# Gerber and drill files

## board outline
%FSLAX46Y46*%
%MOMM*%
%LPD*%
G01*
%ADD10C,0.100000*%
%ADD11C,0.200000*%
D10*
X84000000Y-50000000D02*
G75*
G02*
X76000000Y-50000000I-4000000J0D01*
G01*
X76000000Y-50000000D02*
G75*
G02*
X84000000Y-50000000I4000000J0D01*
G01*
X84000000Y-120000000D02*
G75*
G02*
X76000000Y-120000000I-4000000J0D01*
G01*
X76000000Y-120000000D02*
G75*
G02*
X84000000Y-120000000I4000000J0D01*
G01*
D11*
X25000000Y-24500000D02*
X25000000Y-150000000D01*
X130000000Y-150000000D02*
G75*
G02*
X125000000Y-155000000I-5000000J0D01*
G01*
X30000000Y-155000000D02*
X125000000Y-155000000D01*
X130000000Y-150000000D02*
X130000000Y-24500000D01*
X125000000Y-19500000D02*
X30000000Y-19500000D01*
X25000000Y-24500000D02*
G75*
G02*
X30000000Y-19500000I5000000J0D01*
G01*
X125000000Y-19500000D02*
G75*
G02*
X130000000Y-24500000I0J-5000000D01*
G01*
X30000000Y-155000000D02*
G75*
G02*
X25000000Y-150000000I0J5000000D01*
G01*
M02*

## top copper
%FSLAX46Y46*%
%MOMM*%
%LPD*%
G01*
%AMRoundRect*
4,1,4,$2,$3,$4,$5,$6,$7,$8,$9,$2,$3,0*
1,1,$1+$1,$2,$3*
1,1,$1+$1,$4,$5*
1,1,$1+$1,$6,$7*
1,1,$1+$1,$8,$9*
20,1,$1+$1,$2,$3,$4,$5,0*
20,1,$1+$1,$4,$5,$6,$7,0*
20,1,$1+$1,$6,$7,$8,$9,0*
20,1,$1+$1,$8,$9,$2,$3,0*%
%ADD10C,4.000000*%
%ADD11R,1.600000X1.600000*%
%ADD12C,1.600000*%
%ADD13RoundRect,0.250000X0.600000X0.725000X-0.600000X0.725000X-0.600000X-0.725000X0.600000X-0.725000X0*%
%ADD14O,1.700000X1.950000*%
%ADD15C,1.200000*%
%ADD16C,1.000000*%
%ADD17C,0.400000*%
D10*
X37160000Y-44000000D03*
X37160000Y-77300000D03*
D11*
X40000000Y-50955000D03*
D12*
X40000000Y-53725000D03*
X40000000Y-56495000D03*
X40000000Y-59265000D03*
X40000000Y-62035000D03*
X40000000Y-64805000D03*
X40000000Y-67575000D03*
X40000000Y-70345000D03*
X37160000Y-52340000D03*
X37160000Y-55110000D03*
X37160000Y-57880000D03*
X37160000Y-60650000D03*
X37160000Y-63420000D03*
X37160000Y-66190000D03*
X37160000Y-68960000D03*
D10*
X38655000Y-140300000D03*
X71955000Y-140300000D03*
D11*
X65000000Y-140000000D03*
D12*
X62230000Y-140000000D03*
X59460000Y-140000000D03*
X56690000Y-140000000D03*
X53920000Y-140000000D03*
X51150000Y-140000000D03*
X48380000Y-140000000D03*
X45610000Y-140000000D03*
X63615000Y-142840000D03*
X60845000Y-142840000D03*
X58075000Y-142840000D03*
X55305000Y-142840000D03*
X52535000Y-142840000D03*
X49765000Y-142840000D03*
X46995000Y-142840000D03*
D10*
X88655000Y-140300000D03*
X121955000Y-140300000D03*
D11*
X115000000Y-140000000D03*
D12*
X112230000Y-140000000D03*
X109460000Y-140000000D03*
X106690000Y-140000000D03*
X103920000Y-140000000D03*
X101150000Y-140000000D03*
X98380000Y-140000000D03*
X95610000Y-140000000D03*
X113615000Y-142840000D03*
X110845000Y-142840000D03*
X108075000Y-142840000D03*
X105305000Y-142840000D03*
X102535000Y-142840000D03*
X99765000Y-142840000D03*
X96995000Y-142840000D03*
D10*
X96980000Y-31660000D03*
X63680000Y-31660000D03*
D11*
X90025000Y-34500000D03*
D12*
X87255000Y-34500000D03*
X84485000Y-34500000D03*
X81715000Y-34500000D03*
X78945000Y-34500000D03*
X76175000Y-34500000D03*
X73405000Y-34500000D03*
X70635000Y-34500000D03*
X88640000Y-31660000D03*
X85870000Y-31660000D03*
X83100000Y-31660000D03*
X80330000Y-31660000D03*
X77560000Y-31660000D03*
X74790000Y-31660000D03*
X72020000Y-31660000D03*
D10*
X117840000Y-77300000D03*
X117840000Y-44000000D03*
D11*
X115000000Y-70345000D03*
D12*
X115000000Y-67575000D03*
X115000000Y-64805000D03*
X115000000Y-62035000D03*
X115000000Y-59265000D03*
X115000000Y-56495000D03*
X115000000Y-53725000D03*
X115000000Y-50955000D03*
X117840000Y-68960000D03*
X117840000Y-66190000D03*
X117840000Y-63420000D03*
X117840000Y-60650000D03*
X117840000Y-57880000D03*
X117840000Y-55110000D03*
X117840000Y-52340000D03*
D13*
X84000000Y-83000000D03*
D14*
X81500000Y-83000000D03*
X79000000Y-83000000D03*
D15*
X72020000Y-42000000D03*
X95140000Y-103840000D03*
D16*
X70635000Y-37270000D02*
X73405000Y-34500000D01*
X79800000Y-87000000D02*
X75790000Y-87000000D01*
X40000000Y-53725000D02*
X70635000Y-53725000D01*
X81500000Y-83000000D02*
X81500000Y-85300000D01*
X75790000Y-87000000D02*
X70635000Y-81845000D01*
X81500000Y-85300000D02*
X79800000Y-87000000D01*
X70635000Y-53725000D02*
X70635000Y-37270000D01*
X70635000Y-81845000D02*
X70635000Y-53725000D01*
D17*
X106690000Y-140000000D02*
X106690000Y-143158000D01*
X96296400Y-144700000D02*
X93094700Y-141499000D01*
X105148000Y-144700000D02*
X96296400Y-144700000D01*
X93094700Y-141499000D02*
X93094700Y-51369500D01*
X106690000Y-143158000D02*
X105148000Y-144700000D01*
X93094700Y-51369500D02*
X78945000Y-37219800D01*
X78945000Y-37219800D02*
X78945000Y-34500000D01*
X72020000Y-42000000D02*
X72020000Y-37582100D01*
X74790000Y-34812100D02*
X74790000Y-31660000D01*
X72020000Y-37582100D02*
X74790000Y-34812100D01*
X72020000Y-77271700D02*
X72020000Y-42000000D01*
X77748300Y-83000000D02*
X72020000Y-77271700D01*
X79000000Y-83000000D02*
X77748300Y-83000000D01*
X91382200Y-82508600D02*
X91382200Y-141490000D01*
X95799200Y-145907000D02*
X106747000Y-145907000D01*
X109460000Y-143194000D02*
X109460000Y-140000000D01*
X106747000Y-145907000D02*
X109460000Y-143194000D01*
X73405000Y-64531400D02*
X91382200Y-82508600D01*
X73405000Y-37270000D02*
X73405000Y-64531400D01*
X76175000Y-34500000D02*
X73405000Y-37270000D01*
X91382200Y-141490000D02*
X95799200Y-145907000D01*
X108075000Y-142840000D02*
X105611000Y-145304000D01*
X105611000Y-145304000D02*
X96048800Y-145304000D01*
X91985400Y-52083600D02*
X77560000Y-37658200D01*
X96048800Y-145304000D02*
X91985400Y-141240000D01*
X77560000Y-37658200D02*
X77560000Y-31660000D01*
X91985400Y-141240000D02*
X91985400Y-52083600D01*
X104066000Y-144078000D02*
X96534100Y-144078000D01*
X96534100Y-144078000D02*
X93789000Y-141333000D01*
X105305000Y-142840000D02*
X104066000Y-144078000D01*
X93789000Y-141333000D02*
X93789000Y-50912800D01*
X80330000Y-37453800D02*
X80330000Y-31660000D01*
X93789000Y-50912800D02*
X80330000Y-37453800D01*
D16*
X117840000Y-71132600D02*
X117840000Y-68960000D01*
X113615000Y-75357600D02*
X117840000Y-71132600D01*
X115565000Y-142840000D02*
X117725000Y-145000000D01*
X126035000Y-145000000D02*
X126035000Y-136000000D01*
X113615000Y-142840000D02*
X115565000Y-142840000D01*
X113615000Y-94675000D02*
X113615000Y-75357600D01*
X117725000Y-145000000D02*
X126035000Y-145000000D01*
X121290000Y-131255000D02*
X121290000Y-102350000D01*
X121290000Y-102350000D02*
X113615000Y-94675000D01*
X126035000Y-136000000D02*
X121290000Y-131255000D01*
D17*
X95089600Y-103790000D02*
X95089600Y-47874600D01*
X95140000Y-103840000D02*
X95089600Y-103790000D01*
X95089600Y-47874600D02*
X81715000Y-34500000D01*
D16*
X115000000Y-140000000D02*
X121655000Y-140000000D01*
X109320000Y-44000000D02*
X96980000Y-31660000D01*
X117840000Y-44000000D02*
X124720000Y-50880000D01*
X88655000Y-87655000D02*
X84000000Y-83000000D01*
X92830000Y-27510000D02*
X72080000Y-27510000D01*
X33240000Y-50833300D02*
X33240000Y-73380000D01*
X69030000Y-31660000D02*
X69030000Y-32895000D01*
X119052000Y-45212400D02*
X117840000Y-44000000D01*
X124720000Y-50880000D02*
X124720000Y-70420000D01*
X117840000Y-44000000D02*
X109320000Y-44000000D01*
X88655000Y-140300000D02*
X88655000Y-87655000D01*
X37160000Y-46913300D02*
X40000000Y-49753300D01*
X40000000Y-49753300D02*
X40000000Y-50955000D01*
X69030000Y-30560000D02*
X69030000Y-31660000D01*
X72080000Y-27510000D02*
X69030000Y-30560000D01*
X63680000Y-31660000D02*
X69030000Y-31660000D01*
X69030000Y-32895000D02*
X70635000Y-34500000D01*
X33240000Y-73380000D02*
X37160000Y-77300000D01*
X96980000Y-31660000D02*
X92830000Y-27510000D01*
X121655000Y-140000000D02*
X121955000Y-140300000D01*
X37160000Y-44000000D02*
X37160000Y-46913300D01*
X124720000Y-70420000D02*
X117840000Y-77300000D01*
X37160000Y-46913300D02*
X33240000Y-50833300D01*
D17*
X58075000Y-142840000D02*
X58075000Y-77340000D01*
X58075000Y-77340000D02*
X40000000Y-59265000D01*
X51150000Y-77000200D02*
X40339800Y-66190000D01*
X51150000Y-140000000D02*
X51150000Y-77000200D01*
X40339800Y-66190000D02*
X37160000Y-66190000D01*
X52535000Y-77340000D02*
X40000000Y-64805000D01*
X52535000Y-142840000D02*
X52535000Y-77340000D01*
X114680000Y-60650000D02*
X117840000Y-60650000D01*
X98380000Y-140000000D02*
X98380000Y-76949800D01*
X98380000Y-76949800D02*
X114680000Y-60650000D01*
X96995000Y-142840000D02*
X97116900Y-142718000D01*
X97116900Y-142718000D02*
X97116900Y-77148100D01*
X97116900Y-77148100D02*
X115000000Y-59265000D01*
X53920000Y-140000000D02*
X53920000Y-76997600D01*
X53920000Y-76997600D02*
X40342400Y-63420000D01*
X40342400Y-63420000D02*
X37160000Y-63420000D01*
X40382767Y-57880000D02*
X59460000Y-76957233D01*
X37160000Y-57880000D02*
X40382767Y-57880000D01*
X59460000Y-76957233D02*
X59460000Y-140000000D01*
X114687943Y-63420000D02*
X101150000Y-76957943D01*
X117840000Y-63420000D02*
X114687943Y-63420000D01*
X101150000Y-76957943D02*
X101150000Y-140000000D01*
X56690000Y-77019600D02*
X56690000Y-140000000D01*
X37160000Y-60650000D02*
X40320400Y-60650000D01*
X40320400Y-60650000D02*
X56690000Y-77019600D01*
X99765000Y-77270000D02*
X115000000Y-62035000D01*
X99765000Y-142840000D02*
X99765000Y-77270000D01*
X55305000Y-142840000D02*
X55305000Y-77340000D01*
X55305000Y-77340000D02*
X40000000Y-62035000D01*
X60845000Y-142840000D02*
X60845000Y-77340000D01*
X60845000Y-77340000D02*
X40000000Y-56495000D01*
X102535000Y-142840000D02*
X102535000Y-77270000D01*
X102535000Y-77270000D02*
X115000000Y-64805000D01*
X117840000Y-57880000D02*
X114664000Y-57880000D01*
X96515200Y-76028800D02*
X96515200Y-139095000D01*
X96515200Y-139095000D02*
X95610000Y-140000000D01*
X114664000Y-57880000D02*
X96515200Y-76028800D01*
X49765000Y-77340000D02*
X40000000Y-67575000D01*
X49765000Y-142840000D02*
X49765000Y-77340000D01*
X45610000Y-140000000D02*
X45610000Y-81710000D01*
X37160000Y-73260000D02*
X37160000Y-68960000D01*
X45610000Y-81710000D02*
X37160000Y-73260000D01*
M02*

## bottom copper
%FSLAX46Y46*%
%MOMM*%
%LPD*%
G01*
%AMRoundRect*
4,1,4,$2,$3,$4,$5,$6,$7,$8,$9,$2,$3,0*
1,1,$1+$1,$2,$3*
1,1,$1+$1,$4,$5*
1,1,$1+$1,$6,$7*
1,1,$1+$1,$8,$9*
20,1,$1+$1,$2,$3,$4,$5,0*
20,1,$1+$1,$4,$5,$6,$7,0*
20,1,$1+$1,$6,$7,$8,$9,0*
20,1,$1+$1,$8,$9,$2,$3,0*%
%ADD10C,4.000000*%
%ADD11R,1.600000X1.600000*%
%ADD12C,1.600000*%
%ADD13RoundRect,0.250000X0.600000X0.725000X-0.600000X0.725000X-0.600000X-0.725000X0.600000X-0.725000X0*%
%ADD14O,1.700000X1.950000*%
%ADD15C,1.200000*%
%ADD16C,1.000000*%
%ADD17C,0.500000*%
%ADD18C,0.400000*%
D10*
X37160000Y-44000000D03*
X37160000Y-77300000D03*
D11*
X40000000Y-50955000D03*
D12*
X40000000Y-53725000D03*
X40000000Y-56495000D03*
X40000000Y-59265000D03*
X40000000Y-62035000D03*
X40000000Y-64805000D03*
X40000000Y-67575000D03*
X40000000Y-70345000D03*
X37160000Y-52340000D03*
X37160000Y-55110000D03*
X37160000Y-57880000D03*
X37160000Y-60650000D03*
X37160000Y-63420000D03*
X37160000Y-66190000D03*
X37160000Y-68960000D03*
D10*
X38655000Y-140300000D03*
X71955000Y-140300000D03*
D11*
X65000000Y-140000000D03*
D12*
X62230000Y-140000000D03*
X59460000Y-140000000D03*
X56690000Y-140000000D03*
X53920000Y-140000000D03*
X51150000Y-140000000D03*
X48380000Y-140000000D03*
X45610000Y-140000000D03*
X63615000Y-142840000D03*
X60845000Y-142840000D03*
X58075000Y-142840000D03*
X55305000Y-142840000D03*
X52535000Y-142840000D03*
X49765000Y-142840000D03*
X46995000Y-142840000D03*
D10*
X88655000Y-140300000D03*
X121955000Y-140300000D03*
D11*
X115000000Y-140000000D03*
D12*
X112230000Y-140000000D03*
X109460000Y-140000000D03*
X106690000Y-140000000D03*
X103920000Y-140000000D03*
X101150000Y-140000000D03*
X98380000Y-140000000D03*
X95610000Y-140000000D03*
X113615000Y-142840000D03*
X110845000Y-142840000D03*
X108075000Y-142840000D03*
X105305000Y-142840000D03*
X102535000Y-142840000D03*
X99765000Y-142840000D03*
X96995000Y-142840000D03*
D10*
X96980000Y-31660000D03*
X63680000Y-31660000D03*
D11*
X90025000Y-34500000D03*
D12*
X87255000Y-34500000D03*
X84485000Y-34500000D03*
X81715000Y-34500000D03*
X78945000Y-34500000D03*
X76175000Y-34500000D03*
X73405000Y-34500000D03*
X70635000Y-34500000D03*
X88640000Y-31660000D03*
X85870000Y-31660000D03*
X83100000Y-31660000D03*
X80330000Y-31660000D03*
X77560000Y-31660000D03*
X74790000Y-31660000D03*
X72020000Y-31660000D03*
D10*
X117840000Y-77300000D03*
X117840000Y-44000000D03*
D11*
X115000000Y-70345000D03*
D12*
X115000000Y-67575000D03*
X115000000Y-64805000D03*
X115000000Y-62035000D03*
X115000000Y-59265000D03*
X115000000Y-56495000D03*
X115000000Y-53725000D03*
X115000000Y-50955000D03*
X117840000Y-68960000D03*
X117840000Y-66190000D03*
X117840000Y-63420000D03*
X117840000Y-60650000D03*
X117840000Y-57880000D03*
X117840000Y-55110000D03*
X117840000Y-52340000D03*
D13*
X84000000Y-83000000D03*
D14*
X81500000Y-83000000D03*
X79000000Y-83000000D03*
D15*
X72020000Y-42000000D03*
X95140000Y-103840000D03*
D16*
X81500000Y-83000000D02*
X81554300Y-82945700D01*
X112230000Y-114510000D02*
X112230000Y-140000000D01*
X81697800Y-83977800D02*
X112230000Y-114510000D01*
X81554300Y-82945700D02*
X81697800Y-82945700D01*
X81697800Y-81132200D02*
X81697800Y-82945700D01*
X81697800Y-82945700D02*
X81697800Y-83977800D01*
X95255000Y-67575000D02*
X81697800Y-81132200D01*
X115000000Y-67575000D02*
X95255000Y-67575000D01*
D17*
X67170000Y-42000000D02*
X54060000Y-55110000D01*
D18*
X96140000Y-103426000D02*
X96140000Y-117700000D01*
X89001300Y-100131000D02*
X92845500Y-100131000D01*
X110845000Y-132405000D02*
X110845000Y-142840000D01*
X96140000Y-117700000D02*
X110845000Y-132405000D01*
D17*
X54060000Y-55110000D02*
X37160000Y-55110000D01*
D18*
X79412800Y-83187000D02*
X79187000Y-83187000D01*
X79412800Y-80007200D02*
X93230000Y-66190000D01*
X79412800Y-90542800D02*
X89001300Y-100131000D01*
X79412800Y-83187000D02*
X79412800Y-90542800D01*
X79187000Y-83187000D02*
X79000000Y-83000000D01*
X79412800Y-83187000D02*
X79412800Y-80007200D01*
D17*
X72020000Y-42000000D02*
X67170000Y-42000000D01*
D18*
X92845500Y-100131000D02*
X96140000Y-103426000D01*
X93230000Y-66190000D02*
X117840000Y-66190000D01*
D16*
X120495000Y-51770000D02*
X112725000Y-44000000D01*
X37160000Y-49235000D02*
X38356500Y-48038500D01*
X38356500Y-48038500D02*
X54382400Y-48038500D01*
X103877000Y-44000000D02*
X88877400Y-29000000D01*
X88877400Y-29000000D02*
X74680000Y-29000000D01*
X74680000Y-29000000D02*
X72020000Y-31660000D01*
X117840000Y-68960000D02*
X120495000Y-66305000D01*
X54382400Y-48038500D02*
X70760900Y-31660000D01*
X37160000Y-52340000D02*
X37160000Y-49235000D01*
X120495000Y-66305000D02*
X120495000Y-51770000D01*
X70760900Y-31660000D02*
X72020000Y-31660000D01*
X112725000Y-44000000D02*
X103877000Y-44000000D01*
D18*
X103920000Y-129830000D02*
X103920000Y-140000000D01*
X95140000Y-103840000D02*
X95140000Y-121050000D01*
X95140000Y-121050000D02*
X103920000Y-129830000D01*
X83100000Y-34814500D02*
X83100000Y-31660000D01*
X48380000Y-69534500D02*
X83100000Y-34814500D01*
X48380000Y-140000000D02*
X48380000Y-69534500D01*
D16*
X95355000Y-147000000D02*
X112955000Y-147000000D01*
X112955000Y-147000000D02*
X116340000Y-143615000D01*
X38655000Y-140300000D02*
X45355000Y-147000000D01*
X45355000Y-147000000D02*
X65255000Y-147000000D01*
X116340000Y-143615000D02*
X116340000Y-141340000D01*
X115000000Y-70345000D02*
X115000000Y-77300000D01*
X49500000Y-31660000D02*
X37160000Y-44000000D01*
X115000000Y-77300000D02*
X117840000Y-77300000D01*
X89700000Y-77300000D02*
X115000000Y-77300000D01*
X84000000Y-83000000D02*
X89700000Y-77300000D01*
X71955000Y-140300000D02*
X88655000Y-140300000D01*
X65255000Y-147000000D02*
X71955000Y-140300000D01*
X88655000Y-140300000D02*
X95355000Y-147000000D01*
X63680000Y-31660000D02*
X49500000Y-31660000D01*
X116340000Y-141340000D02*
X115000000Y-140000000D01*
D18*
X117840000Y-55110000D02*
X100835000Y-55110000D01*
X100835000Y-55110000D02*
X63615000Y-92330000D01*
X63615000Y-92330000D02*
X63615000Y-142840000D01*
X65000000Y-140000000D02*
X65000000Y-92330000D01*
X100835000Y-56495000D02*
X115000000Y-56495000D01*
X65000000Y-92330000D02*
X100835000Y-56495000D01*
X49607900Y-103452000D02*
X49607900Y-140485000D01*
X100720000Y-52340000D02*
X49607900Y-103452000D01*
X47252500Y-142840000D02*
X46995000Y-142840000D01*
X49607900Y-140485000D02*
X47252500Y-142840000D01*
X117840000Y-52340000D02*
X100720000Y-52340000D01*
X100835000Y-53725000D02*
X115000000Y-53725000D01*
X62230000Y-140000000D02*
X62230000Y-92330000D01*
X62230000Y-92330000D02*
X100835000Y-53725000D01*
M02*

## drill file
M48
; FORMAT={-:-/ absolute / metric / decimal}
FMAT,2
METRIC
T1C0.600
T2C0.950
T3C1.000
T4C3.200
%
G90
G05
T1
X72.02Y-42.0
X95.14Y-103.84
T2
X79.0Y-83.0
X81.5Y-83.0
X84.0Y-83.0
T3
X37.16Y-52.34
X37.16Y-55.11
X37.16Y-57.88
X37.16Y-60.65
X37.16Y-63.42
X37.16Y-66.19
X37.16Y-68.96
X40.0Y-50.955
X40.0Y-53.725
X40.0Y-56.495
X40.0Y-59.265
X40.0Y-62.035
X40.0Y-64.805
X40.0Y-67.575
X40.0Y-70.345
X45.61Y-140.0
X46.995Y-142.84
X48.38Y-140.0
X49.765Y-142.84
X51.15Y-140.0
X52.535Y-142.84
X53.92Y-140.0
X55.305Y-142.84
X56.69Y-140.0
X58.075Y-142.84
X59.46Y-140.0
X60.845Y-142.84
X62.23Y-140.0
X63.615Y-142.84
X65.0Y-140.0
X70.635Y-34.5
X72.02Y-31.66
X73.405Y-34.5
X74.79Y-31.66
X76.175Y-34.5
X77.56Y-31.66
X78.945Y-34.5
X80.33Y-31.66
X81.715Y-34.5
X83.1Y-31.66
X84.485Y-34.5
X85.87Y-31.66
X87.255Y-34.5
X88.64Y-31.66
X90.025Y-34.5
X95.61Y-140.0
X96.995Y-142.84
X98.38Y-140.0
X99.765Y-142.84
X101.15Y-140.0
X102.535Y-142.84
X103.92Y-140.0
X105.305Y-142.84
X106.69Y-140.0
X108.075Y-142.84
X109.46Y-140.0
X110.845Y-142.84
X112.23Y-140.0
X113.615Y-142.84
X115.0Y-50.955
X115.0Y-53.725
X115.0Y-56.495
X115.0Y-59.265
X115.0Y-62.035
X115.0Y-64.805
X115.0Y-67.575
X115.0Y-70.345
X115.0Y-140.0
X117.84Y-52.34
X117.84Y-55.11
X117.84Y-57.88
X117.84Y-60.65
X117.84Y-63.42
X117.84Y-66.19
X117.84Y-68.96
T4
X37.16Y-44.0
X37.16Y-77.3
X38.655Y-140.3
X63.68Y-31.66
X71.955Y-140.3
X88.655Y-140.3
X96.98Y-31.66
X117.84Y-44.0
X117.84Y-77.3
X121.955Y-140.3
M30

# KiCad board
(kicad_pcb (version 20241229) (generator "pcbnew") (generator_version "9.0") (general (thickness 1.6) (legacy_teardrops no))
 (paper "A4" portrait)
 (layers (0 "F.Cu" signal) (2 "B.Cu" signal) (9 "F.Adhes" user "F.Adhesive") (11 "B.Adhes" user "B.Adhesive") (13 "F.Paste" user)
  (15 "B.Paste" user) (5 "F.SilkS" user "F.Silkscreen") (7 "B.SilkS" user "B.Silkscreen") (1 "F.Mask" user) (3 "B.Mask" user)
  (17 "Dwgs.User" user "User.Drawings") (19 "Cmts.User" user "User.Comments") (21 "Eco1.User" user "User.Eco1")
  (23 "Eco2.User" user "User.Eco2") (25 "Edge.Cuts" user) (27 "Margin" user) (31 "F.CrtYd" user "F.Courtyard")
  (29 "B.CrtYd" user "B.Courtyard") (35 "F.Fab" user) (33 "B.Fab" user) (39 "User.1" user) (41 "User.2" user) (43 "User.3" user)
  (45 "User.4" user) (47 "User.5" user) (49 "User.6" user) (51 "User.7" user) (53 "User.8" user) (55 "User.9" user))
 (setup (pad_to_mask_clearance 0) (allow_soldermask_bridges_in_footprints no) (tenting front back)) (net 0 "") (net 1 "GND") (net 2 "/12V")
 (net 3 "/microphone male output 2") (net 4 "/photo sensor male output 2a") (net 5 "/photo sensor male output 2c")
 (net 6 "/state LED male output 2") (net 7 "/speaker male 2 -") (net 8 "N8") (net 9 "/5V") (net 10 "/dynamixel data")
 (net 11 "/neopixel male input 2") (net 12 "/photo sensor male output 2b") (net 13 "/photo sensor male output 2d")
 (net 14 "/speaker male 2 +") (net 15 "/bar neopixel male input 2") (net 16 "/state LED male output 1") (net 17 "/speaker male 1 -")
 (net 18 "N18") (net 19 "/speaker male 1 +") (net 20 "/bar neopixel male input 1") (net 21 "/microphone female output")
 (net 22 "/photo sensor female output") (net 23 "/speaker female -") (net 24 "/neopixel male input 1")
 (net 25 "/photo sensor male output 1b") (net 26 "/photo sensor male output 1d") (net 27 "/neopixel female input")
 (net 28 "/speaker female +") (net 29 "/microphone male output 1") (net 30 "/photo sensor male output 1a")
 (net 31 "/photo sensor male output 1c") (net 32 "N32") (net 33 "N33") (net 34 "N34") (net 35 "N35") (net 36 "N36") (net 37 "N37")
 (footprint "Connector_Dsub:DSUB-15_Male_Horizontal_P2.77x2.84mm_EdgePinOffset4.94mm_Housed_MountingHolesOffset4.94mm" (layer "F.Cu")
  (at 40 50.955 -90)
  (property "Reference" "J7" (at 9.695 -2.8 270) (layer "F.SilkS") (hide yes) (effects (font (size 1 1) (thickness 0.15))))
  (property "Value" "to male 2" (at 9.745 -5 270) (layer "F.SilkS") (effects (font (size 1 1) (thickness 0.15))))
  (pad "0" thru_hole circle (at -6.955 2.84 270) (size 4 4) (drill 3.2) (layers "*.Cu" "*.Mask") (remove_unused_layers no) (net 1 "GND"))
  (pad "0" thru_hole circle (at 26.345 2.84 270) (size 4 4) (drill 3.2) (layers "*.Cu" "*.Mask") (remove_unused_layers no) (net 1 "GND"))
  (pad "1" thru_hole rect (at 0 0 270) (size 1.6 1.6) (drill 1) (layers "*.Cu" "*.Mask") (remove_unused_layers no) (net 1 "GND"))
  (pad "2" thru_hole circle (at 2.77 0 270) (size 1.6 1.6) (drill 1) (layers "*.Cu" "*.Mask") (remove_unused_layers no) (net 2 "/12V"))
  (pad "3" thru_hole circle (at 5.54 0 270) (size 1.6 1.6) (drill 1) (layers "*.Cu" "*.Mask") (remove_unused_layers no)
   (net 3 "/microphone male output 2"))
  (pad "4" thru_hole circle (at 8.31 0 270) (size 1.6 1.6) (drill 1) (layers "*.Cu" "*.Mask") (remove_unused_layers no)
   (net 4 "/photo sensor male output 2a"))
  (pad "5" thru_hole circle (at 11.08 0 270) (size 1.6 1.6) (drill 1) (layers "*.Cu" "*.Mask") (remove_unused_layers no)
   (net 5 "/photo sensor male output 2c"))
  (pad "6" thru_hole circle (at 13.85 0 270) (size 1.6 1.6) (drill 1) (layers "*.Cu" "*.Mask") (remove_unused_layers no)
   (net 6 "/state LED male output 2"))
  (pad "7" thru_hole circle (at 16.62 0 270) (size 1.6 1.6) (drill 1) (layers "*.Cu" "*.Mask") (remove_unused_layers no)
   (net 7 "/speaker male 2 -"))
  (pad "8" thru_hole circle (at 19.39 0 270) (size 1.6 1.6) (drill 1) (layers "*.Cu" "*.Mask") (remove_unused_layers no) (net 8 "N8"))
  (pad "9" thru_hole circle (at 1.385 2.84 270) (size 1.6 1.6) (drill 1) (layers "*.Cu" "*.Mask") (remove_unused_layers no) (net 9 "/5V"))
  (pad "10" thru_hole circle (at 4.155 2.84 270) (size 1.6 1.6) (drill 1) (layers "*.Cu" "*.Mask") (remove_unused_layers no)
   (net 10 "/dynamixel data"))
  (pad "11" thru_hole circle (at 6.925 2.84 270) (size 1.6 1.6) (drill 1) (layers "*.Cu" "*.Mask") (remove_unused_layers no)
   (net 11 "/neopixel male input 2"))
  (pad "12" thru_hole circle (at 9.695 2.84 270) (size 1.6 1.6) (drill 1) (layers "*.Cu" "*.Mask") (remove_unused_layers no)
   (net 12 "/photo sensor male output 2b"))
  (pad "13" thru_hole circle (at 12.465 2.84 270) (size 1.6 1.6) (drill 1) (layers "*.Cu" "*.Mask") (remove_unused_layers no)
   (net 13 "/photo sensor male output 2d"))
  (pad "14" thru_hole circle (at 15.235 2.84 270) (size 1.6 1.6) (drill 1) (layers "*.Cu" "*.Mask") (remove_unused_layers no)
   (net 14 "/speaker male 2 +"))
  (pad "15" thru_hole circle (at 18.005 2.84 270) (size 1.6 1.6) (drill 1) (layers "*.Cu" "*.Mask") (remove_unused_layers no)
   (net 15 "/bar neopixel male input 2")))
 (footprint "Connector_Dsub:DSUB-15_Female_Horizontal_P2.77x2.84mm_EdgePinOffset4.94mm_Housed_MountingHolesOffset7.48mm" (layer "F.Cu")
  (at 65 140)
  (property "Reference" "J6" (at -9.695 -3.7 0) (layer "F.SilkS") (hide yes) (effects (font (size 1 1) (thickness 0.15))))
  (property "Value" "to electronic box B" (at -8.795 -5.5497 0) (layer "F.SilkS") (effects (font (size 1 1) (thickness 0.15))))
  (pad "0" thru_hole circle (at -26.345 0.3) (size 4 4) (drill 3.2) (layers "*.Cu" "*.Mask") (remove_unused_layers no) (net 1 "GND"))
  (pad "0" thru_hole circle (at 6.955 0.3) (size 4 4) (drill 3.2) (layers "*.Cu" "*.Mask") (remove_unused_layers no) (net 1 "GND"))
  (pad "1" thru_hole rect (at 0 0) (size 1.6 1.6) (drill 1) (layers "*.Cu" "*.Mask") (remove_unused_layers no)
   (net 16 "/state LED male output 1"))
  (pad "2" thru_hole circle (at -2.77 0) (size 1.6 1.6) (drill 1) (layers "*.Cu" "*.Mask") (remove_unused_layers no)
   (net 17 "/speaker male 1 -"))
  (pad "3" thru_hole circle (at -5.54 0) (size 1.6 1.6) (drill 1) (layers "*.Cu" "*.Mask") (remove_unused_layers no)
   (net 11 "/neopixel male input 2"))
  (pad "4" thru_hole circle (at -8.31 0) (size 1.6 1.6) (drill 1) (layers "*.Cu" "*.Mask") (remove_unused_layers no)
   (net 12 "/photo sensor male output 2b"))
  (pad "5" thru_hole circle (at -11.08 0) (size 1.6 1.6) (drill 1) (layers "*.Cu" "*.Mask") (remove_unused_layers no)
   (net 13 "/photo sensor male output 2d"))
  (pad "6" thru_hole circle (at -13.85 0) (size 1.6 1.6) (drill 1) (layers "*.Cu" "*.Mask") (remove_unused_layers no)
   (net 14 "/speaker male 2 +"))
  (pad "7" thru_hole circle (at -16.62 0) (size 1.6 1.6) (drill 1) (layers "*.Cu" "*.Mask") (remove_unused_layers no) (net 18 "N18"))
  (pad "8" thru_hole circle (at -19.39 0) (size 1.6 1.6) (drill 1) (layers "*.Cu" "*.Mask") (remove_unused_layers no)
   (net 15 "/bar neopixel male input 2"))
  (pad "9" thru_hole circle (at -1.385 2.84) (size 1.6 1.6) (drill 1) (layers "*.Cu" "*.Mask") (remove_unused_layers no)
   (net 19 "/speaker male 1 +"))
  (pad "10" thru_hole circle (at -4.155 2.84) (size 1.6 1.6) (drill 1) (layers "*.Cu" "*.Mask") (remove_unused_layers no)
   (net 3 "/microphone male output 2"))
  (pad "11" thru_hole circle (at -6.925 2.84) (size 1.6 1.6) (drill 1) (layers "*.Cu" "*.Mask") (remove_unused_layers no)
   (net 4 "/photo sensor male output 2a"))
  (pad "12" thru_hole circle (at -9.695 2.84) (size 1.6 1.6) (drill 1) (layers "*.Cu" "*.Mask") (remove_unused_layers no)
   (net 5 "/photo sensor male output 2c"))
  (pad "13" thru_hole circle (at -12.465 2.84) (size 1.6 1.6) (drill 1) (layers "*.Cu" "*.Mask") (remove_unused_layers no)
   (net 6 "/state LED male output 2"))
  (pad "14" thru_hole circle (at -15.235 2.84) (size 1.6 1.6) (drill 1) (layers "*.Cu" "*.Mask") (remove_unused_layers no)
   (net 7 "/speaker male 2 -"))
  (pad "15" thru_hole circle (at -18.005 2.84) (size 1.6 1.6) (drill 1) (layers "*.Cu" "*.Mask") (remove_unused_layers no)
   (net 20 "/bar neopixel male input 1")))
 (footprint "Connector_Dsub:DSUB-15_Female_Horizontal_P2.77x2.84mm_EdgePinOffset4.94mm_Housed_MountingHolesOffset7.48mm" (layer "F.Cu")
  (at 115 140)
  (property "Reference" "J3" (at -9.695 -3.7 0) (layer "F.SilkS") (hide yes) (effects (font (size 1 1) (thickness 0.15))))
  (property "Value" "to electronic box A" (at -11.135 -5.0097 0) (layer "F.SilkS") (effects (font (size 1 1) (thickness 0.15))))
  (pad "0" thru_hole circle (at -26.345 0.3) (size 4 4) (drill 3.2) (layers "*.Cu" "*.Mask") (remove_unused_layers no) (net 1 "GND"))
  (pad "0" thru_hole circle (at 6.955 0.3) (size 4 4) (drill 3.2) (layers "*.Cu" "*.Mask") (remove_unused_layers no) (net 1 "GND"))
  (pad "1" thru_hole rect (at 0 0) (size 1.6 1.6) (drill 1) (layers "*.Cu" "*.Mask") (remove_unused_layers no) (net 1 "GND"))
  (pad "2" thru_hole circle (at -2.77 0) (size 1.6 1.6) (drill 1) (layers "*.Cu" "*.Mask") (remove_unused_layers no) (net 2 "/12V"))
  (pad "3" thru_hole circle (at -5.54 0) (size 1.6 1.6) (drill 1) (layers "*.Cu" "*.Mask") (remove_unused_layers no)
   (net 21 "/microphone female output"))
  (pad "4" thru_hole circle (at -8.31 0) (size 1.6 1.6) (drill 1) (layers "*.Cu" "*.Mask") (remove_unused_layers no)
   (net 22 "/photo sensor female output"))
  (pad "5" thru_hole circle (at -11.08 0) (size 1.6 1.6) (drill 1) (layers "*.Cu" "*.Mask") (remove_unused_layers no)
   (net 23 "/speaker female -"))
  (pad "6" thru_hole circle (at -13.85 0) (size 1.6 1.6) (drill 1) (layers "*.Cu" "*.Mask") (remove_unused_layers no)
   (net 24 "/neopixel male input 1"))
  (pad "7" thru_hole circle (at -16.62 0) (size 1.6 1.6) (drill 1) (layers "*.Cu" "*.Mask") (remove_unused_layers no)
   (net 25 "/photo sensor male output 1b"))
  (pad "8" thru_hole circle (at -19.39 0) (size 1.6 1.6) (drill 1) (layers "*.Cu" "*.Mask") (remove_unused_layers no)
   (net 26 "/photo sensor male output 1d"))
  (pad "9" thru_hole circle (at -1.385 2.84) (size 1.6 1.6) (drill 1) (layers "*.Cu" "*.Mask") (remove_unused_layers no) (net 9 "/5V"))
  (pad "10" thru_hole circle (at -4.155 2.84) (size 1.6 1.6) (drill 1) (layers "*.Cu" "*.Mask") (remove_unused_layers no)
   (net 10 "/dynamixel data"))
  (pad "11" thru_hole circle (at -6.925 2.84) (size 1.6 1.6) (drill 1) (layers "*.Cu" "*.Mask") (remove_unused_layers no)
   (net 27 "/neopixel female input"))
  (pad "12" thru_hole circle (at -9.695 2.84) (size 1.6 1.6) (drill 1) (layers "*.Cu" "*.Mask") (remove_unused_layers no)
   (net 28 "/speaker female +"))
  (pad "13" thru_hole circle (at -12.465 2.84) (size 1.6 1.6) (drill 1) (layers "*.Cu" "*.Mask") (remove_unused_layers no)
   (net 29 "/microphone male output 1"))
  (pad "14" thru_hole circle (at -15.235 2.84) (size 1.6 1.6) (drill 1) (layers "*.Cu" "*.Mask") (remove_unused_layers no)
   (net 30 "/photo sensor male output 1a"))
  (pad "15" thru_hole circle (at -18.005 2.84) (size 1.6 1.6) (drill 1) (layers "*.Cu" "*.Mask") (remove_unused_layers no)
   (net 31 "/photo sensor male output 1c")))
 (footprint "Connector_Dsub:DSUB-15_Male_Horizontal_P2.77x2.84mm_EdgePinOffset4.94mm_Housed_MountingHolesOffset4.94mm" (layer "F.Cu")
  (at 90.025 34.5 180)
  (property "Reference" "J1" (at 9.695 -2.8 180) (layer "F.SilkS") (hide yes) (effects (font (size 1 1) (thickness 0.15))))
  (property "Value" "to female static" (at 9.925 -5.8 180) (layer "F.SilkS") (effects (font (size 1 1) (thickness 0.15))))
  (pad "0" thru_hole circle (at -6.955 2.84 180) (size 4 4) (drill 3.2) (layers "*.Cu" "*.Mask") (remove_unused_layers no) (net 1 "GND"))
  (pad "0" thru_hole circle (at 26.345 2.84 180) (size 4 4) (drill 3.2) (layers "*.Cu" "*.Mask") (remove_unused_layers no) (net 1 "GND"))
  (pad "1" thru_hole rect (at 0 0 180) (size 1.6 1.6) (drill 1) (layers "*.Cu" "*.Mask") (remove_unused_layers no) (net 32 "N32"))
  (pad "2" thru_hole circle (at 2.77 0 180) (size 1.6 1.6) (drill 1) (layers "*.Cu" "*.Mask") (remove_unused_layers no) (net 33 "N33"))
  (pad "3" thru_hole circle (at 5.54 0 180) (size 1.6 1.6) (drill 1) (layers "*.Cu" "*.Mask") (remove_unused_layers no) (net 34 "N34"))
  (pad "4" thru_hole circle (at 8.31 0 180) (size 1.6 1.6) (drill 1) (layers "*.Cu" "*.Mask") (remove_unused_layers no)
   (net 23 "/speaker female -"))
  (pad "5" thru_hole circle (at 11.08 0 180) (size 1.6 1.6) (drill 1) (layers "*.Cu" "*.Mask") (remove_unused_layers no)
   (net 22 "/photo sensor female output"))
  (pad "6" thru_hole circle (at 13.85 0 180) (size 1.6 1.6) (drill 1) (layers "*.Cu" "*.Mask") (remove_unused_layers no)
   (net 21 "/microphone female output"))
  (pad "7" thru_hole circle (at 16.62 0 180) (size 1.6 1.6) (drill 1) (layers "*.Cu" "*.Mask") (remove_unused_layers no) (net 2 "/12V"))
  (pad "8" thru_hole circle (at 19.39 0 180) (size 1.6 1.6) (drill 1) (layers "*.Cu" "*.Mask") (remove_unused_layers no) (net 1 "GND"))
  (pad "9" thru_hole circle (at 1.385 2.84 180) (size 1.6 1.6) (drill 1) (layers "*.Cu" "*.Mask") (remove_unused_layers no) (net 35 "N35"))
  (pad "10" thru_hole circle (at 4.155 2.84 180) (size 1.6 1.6) (drill 1) (layers "*.Cu" "*.Mask") (remove_unused_layers no) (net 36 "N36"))
  (pad "11" thru_hole circle (at 6.925 2.84 180) (size 1.6 1.6) (drill 1) (layers "*.Cu" "*.Mask") (remove_unused_layers no) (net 18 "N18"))
  (pad "12" thru_hole circle (at 9.695 2.84 180) (size 1.6 1.6) (drill 1) (layers "*.Cu" "*.Mask") (remove_unused_layers no)
   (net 28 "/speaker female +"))
  (pad "13" thru_hole circle (at 12.465 2.84 180) (size 1.6 1.6) (drill 1) (layers "*.Cu" "*.Mask") (remove_unused_layers no)
   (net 27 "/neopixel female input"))
  (pad "14" thru_hole circle (at 15.235 2.84 180) (size 1.6 1.6) (drill 1) (layers "*.Cu" "*.Mask") (remove_unused_layers no)
   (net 10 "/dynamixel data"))
  (pad "15" thru_hole circle (at 18.005 2.84 180) (size 1.6 1.6) (drill 1) (layers "*.Cu" "*.Mask") (remove_unused_layers no) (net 9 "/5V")))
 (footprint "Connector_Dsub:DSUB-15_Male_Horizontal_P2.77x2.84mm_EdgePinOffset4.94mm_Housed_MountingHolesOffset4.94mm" (layer "F.Cu")
  (at 115 70.345 90)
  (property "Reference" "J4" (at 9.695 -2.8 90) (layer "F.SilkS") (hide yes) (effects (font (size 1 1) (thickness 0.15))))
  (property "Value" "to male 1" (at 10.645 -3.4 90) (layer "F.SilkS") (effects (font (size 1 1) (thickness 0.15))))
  (pad "0" thru_hole circle (at -6.955 2.84 90) (size 4 4) (drill 3.2) (layers "*.Cu" "*.Mask") (remove_unused_layers no) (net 1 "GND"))
  (pad "0" thru_hole circle (at 26.345 2.84 90) (size 4 4) (drill 3.2) (layers "*.Cu" "*.Mask") (remove_unused_layers no) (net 1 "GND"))
  (pad "1" thru_hole rect (at 0 0 90) (size 1.6 1.6) (drill 1) (layers "*.Cu" "*.Mask") (remove_unused_layers no) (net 1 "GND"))
  (pad "2" thru_hole circle (at 2.77 0 90) (size 1.6 1.6) (drill 1) (layers "*.Cu" "*.Mask") (remove_unused_layers no) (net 2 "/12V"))
  (pad "3" thru_hole circle (at 5.54 0 90) (size 1.6 1.6) (drill 1) (layers "*.Cu" "*.Mask") (remove_unused_layers no)
   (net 29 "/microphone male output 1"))
  (pad "4" thru_hole circle (at 8.31 0 90) (size 1.6 1.6) (drill 1) (layers "*.Cu" "*.Mask") (remove_unused_layers no)
   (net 30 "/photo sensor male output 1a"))
  (pad "5" thru_hole circle (at 11.08 0 90) (size 1.6 1.6) (drill 1) (layers "*.Cu" "*.Mask") (remove_unused_layers no)
   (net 31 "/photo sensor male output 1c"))
  (pad "6" thru_hole circle (at 13.85 0 90) (size 1.6 1.6) (drill 1) (layers "*.Cu" "*.Mask") (remove_unused_layers no)
   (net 16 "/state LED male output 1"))
  (pad "7" thru_hole circle (at 16.62 0 90) (size 1.6 1.6) (drill 1) (layers "*.Cu" "*.Mask") (remove_unused_layers no)
   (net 17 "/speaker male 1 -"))
  (pad "8" thru_hole circle (at 19.39 0 90) (size 1.6 1.6) (drill 1) (layers "*.Cu" "*.Mask") (remove_unused_layers no) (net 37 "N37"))
  (pad "9" thru_hole circle (at 1.385 2.84 90) (size 1.6 1.6) (drill 1) (layers "*.Cu" "*.Mask") (remove_unused_layers no) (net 9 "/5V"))
  (pad "10" thru_hole circle (at 4.155 2.84 90) (size 1.6 1.6) (drill 1) (layers "*.Cu" "*.Mask") (remove_unused_layers no)
   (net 10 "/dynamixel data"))
  (pad "11" thru_hole circle (at 6.925 2.84 90) (size 1.6 1.6) (drill 1) (layers "*.Cu" "*.Mask") (remove_unused_layers no)
   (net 24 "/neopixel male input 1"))
  (pad "12" thru_hole circle (at 9.695 2.84 90) (size 1.6 1.6) (drill 1) (layers "*.Cu" "*.Mask") (remove_unused_layers no)
   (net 25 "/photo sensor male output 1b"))
  (pad "13" thru_hole circle (at 12.465 2.84 90) (size 1.6 1.6) (drill 1) (layers "*.Cu" "*.Mask") (remove_unused_layers no)
   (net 26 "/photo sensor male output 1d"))
  (pad "14" thru_hole circle (at 15.235 2.84 90) (size 1.6 1.6) (drill 1) (layers "*.Cu" "*.Mask") (remove_unused_layers no)
   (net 19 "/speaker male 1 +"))
  (pad "15" thru_hole circle (at 18.005 2.84 90) (size 1.6 1.6) (drill 1) (layers "*.Cu" "*.Mask") (remove_unused_layers no)
   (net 20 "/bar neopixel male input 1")))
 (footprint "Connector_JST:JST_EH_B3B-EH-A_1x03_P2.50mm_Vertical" (layer "F.Cu") (at 84 83 180)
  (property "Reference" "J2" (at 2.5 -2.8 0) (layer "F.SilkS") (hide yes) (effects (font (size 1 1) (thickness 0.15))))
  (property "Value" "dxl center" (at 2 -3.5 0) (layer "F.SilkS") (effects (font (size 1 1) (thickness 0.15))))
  (pad "1" thru_hole roundrect (at 0 0 180) (size 1.7 1.95) (drill 0.95) (layers "*.Cu" "*.Mask") (remove_unused_layers no)
   (roundrect_rratio 0.147059) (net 1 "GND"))
  (pad "2" thru_hole oval (at 2.5 0 180) (size 1.7 1.95) (drill 0.95) (layers "*.Cu" "*.Mask") (remove_unused_layers no) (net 2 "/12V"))
  (pad "3" thru_hole oval (at 5 0 180) (size 1.7 1.95) (drill 0.95) (layers "*.Cu" "*.Mask") (remove_unused_layers no)
   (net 10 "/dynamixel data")))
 (gr_circle (center 80 50) (end 84 50) (stroke (width 0.1) (type default)) (fill no) (layer "Edge.Cuts"))
 (gr_circle (center 80 120) (end 84 120) (stroke (width 0.1) (type default)) (fill no) (layer "Edge.Cuts"))
 (gr_line (start 25 24.5) (end 25 150) (stroke (width 0.2) (type default)) (layer "Edge.Cuts"))
 (gr_arc (start 130 150) (mid 128.535534 153.535534) (end 125 155) (stroke (width 0.2) (type default)) (layer "Edge.Cuts"))
 (gr_line (start 30 155) (end 125 155) (stroke (width 0.2) (type default)) (layer "Edge.Cuts"))
 (gr_line (start 130 150) (end 130 24.5) (stroke (width 0.2) (type default)) (layer "Edge.Cuts"))
 (gr_line (start 125 19.5) (end 30 19.5) (stroke (width 0.2) (type default)) (layer "Edge.Cuts"))
 (gr_arc (start 25 24.5) (mid 26.464466 20.964466) (end 30 19.5) (stroke (width 0.2) (type default)) (layer "Edge.Cuts"))
 (gr_arc (start 125 19.5) (mid 128.535534 20.964466) (end 130 24.5) (stroke (width 0.2) (type default)) (layer "Edge.Cuts"))
 (gr_arc (start 30 155) (mid 26.464466 153.535534) (end 25 150) (stroke (width 0.2) (type default)) (layer "Edge.Cuts"))
 (segment (start 70.635 37.27) (end 73.405 34.5) (width 1) (layer "F.Cu") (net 2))
 (segment (start 79.8 87) (end 75.79 87) (width 1) (layer "F.Cu") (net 2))
 (segment (start 40 53.725) (end 70.635 53.725) (width 1) (layer "F.Cu") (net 2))
 (segment (start 81.5 83) (end 81.5 85.3) (width 1) (layer "F.Cu") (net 2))
 (segment (start 75.79 87) (end 70.635 81.845) (width 1) (layer "F.Cu") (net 2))
 (segment (start 81.5 85.3) (end 79.8 87) (width 1) (layer "F.Cu") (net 2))
 (segment (start 70.635 53.725) (end 70.635 37.27) (width 1) (layer "F.Cu") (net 2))
 (segment (start 70.635 81.845) (end 70.635 53.725) (width 1) (layer "F.Cu") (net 2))
 (segment (start 81.5 83) (end 81.5543 82.9457) (width 1) (layer "B.Cu") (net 2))
 (segment (start 112.23 114.51) (end 112.23 140) (width 1) (layer "B.Cu") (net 2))
 (segment (start 81.6978 83.9778) (end 112.23 114.51) (width 1) (layer "B.Cu") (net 2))
 (segment (start 81.5543 82.9457) (end 81.6978 82.9457) (width 1) (layer "B.Cu") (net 2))
 (segment (start 81.6978 81.1322) (end 81.6978 82.9457) (width 1) (layer "B.Cu") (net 2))
 (segment (start 81.6978 82.9457) (end 81.6978 83.9778) (width 1) (layer "B.Cu") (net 2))
 (segment (start 95.255 67.575) (end 81.6978 81.1322) (width 1) (layer "B.Cu") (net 2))
 (segment (start 115 67.575) (end 95.255 67.575) (width 1) (layer "B.Cu") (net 2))
 (segment (start 106.69 140) (end 106.69 143.158) (width 0.4) (layer "F.Cu") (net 22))
 (segment (start 96.2964 144.7) (end 93.0947 141.499) (width 0.4) (layer "F.Cu") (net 22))
 (segment (start 105.148 144.7) (end 96.2964 144.7) (width 0.4) (layer "F.Cu") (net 22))
 (segment (start 93.0947 141.499) (end 93.0947 51.3695) (width 0.4) (layer "F.Cu") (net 22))
 (segment (start 106.69 143.158) (end 105.148 144.7) (width 0.4) (layer "F.Cu") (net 22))
 (segment (start 93.0947 51.3695) (end 78.945 37.2198) (width 0.4) (layer "F.Cu") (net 22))
 (segment (start 78.945 37.2198) (end 78.945 34.5) (width 0.4) (layer "F.Cu") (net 22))
 (segment (start 72.02 42) (end 72.02 37.5821) (width 0.4) (layer "F.Cu") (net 10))
 (segment (start 74.79 34.8121) (end 74.79 31.66) (width 0.4) (layer "F.Cu") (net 10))
 (segment (start 72.02 37.5821) (end 74.79 34.8121) (width 0.4) (layer "F.Cu") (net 10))
 (segment (start 72.02 77.2717) (end 72.02 42) (width 0.4) (layer "F.Cu") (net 10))
 (segment (start 77.7483 83) (end 72.02 77.2717) (width 0.4) (layer "F.Cu") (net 10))
 (segment (start 79 83) (end 77.7483 83) (width 0.4) (layer "F.Cu") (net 10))
 (via (at 72.02 42) (size 1.2) (drill 0.6) (layers "F.Cu" "B.Cu") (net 10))
 (segment (start 67.17 42) (end 54.06 55.11) (width 0.5) (layer "B.Cu") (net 10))
 (segment (start 96.14 103.426) (end 96.14 117.7) (width 0.4) (layer "B.Cu") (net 10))
 (segment (start 89.0013 100.131) (end 92.8455 100.131) (width 0.4) (layer "B.Cu") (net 10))
 (segment (start 110.845 132.405) (end 110.845 142.84) (width 0.4) (layer "B.Cu") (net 10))
 (segment (start 96.14 117.7) (end 110.845 132.405) (width 0.4) (layer "B.Cu") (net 10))
 (segment (start 54.06 55.11) (end 37.16 55.11) (width 0.5) (layer "B.Cu") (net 10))
 (segment (start 79.4128 83.187) (end 79.187 83.187) (width 0.4) (layer "B.Cu") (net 10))
 (segment (start 79.4128 80.0072) (end 93.23 66.19) (width 0.4) (layer "B.Cu") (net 10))
 (segment (start 79.4128 90.5428) (end 89.0013 100.131) (width 0.4) (layer "B.Cu") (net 10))
 (segment (start 79.4128 83.187) (end 79.4128 90.5428) (width 0.4) (layer "B.Cu") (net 10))
 (segment (start 79.187 83.187) (end 79 83) (width 0.4) (layer "B.Cu") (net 10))
 (segment (start 79.4128 83.187) (end 79.4128 80.0072) (width 0.4) (layer "B.Cu") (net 10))
 (segment (start 72.02 42) (end 67.17 42) (width 0.5) (layer "B.Cu") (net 10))
 (segment (start 92.8455 100.131) (end 96.14 103.426) (width 0.4) (layer "B.Cu") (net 10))
 (segment (start 93.23 66.19) (end 117.84 66.19) (width 0.4) (layer "B.Cu") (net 10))
 (segment (start 91.3822 82.5086) (end 91.3822 141.49) (width 0.4) (layer "F.Cu") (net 21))
 (segment (start 95.7992 145.907) (end 106.747 145.907) (width 0.4) (layer "F.Cu") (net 21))
 (segment (start 109.46 143.194) (end 109.46 140) (width 0.4) (layer "F.Cu") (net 21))
 (segment (start 106.747 145.907) (end 109.46 143.194) (width 0.4) (layer "F.Cu") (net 21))
 (segment (start 73.405 64.5314) (end 91.3822 82.5086) (width 0.4) (layer "F.Cu") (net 21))
 (segment (start 73.405 37.27) (end 73.405 64.5314) (width 0.4) (layer "F.Cu") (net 21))
 (segment (start 76.175 34.5) (end 73.405 37.27) (width 0.4) (layer "F.Cu") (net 21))
 (segment (start 91.3822 141.49) (end 95.7992 145.907) (width 0.4) (layer "F.Cu") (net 21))
 (segment (start 108.075 142.84) (end 105.611 145.304) (width 0.4) (layer "F.Cu") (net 27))
 (segment (start 105.611 145.304) (end 96.0488 145.304) (width 0.4) (layer "F.Cu") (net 27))
 (segment (start 91.9854 52.0836) (end 77.56 37.6582) (width 0.4) (layer "F.Cu") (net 27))
 (segment (start 96.0488 145.304) (end 91.9854 141.24) (width 0.4) (layer "F.Cu") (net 27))
 (segment (start 77.56 37.6582) (end 77.56 31.66) (width 0.4) (layer "F.Cu") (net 27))
 (segment (start 91.9854 141.24) (end 91.9854 52.0836) (width 0.4) (layer "F.Cu") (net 27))
 (segment (start 104.066 144.078) (end 96.5341 144.078) (width 0.4) (layer "F.Cu") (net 28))
 (segment (start 96.5341 144.078) (end 93.789 141.333) (width 0.4) (layer "F.Cu") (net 28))
 (segment (start 105.305 142.84) (end 104.066 144.078) (width 0.4) (layer "F.Cu") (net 28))
 (segment (start 93.789 141.333) (end 93.789 50.9128) (width 0.4) (layer "F.Cu") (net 28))
 (segment (start 80.33 37.4538) (end 80.33 31.66) (width 0.4) (layer "F.Cu") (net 28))
 (segment (start 93.789 50.9128) (end 80.33 37.4538) (width 0.4) (layer "F.Cu") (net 28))
 (segment (start 117.84 71.1326) (end 117.84 68.96) (width 1) (layer "F.Cu") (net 9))
 (segment (start 113.615 75.3576) (end 117.84 71.1326) (width 1) (layer "F.Cu") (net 9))
 (segment (start 115.565 142.84) (end 117.725 145) (width 1) (layer "F.Cu") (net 9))
 (segment (start 126.035 145) (end 126.035 136) (width 1) (layer "F.Cu") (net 9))
 (segment (start 113.615 142.84) (end 115.565 142.84) (width 1) (layer "F.Cu") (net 9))
 (segment (start 113.615 94.675) (end 113.615 75.3576) (width 1) (layer "F.Cu") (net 9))
 (segment (start 117.725 145) (end 126.035 145) (width 1) (layer "F.Cu") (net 9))
 (segment (start 121.29 131.255) (end 121.29 102.35) (width 1) (layer "F.Cu") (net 9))
 (segment (start 121.29 102.35) (end 113.615 94.675) (width 1) (layer "F.Cu") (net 9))
 (segment (start 126.035 136) (end 121.29 131.255) (width 1) (layer "F.Cu") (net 9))
 (segment (start 120.495 51.77) (end 112.725 44) (width 1) (layer "B.Cu") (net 9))
 (segment (start 37.16 49.235) (end 38.3565 48.0385) (width 1) (layer "B.Cu") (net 9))
 (segment (start 38.3565 48.0385) (end 54.3824 48.0385) (width 1) (layer "B.Cu") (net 9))
 (segment (start 103.877 44) (end 88.8774 29) (width 1) (layer "B.Cu") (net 9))
 (segment (start 88.8774 29) (end 74.68 29) (width 1) (layer "B.Cu") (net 9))
 (segment (start 74.68 29) (end 72.02 31.66) (width 1) (layer "B.Cu") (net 9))
 (segment (start 117.84 68.96) (end 120.495 66.305) (width 1) (layer "B.Cu") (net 9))
 (segment (start 54.3824 48.0385) (end 70.7609 31.66) (width 1) (layer "B.Cu") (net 9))
 (segment (start 37.16 52.34) (end 37.16 49.235) (width 1) (layer "B.Cu") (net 9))
 (segment (start 120.495 66.305) (end 120.495 51.77) (width 1) (layer "B.Cu") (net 9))
 (segment (start 70.7609 31.66) (end 72.02 31.66) (width 1) (layer "B.Cu") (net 9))
 (segment (start 112.725 44) (end 103.877 44) (width 1) (layer "B.Cu") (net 9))
 (segment (start 95.0896 103.79) (end 95.0896 47.8746) (width 0.4) (layer "F.Cu") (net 23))
 (segment (start 95.14 103.84) (end 95.0896 103.79) (width 0.4) (layer "F.Cu") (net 23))
 (segment (start 95.0896 47.8746) (end 81.715 34.5) (width 0.4) (layer "F.Cu") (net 23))
 (via (at 95.14 103.84) (size 1.2) (drill 0.6) (layers "F.Cu" "B.Cu") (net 23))
 (segment (start 103.92 129.83) (end 103.92 140) (width 0.4) (layer "B.Cu") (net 23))
 (segment (start 95.14 103.84) (end 95.14 121.05) (width 0.4) (layer "B.Cu") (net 23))
 (segment (start 95.14 121.05) (end 103.92 129.83) (width 0.4) (layer "B.Cu") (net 23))
 (segment (start 83.1 34.8145) (end 83.1 31.66) (width 0.4) (layer "B.Cu") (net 18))
 (segment (start 48.38 69.5345) (end 83.1 34.8145) (width 0.4) (layer "B.Cu") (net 18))
 (segment (start 48.38 140) (end 48.38 69.5345) (width 0.4) (layer "B.Cu") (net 18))
 (segment (start 115 140) (end 121.655 140) (width 1) (layer "F.Cu") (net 1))
 (segment (start 109.32 44) (end 96.98 31.66) (width 1) (layer "F.Cu") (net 1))
 (segment (start 117.84 44) (end 124.72 50.88) (width 1) (layer "F.Cu") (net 1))
 (segment (start 88.655 87.655) (end 84 83) (width 1) (layer "F.Cu") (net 1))
 (segment (start 92.83 27.51) (end 72.08 27.51) (width 1) (layer "F.Cu") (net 1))
 (segment (start 33.24 50.8333) (end 33.24 73.38) (width 1) (layer "F.Cu") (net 1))
 (segment (start 69.03 31.66) (end 69.03 32.895) (width 1) (layer "F.Cu") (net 1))
 (segment (start 119.052 45.2124) (end 117.84 44) (width 1) (layer "F.Cu") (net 1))
 (segment (start 124.72 50.88) (end 124.72 70.42) (width 1) (layer "F.Cu") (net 1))
 (segment (start 117.84 44) (end 109.32 44) (width 1) (layer "F.Cu") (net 1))
 (segment (start 88.655 140.3) (end 88.655 87.655) (width 1) (layer "F.Cu") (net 1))
 (segment (start 37.16 46.9133) (end 40 49.7533) (width 1) (layer "F.Cu") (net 1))
 (segment (start 40 49.7533) (end 40 50.955) (width 1) (layer "F.Cu") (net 1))
 (segment (start 69.03 30.56) (end 69.03 31.66) (width 1) (layer "F.Cu") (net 1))
 (segment (start 72.08 27.51) (end 69.03 30.56) (width 1) (layer "F.Cu") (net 1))
 (segment (start 63.68 31.66) (end 69.03 31.66) (width 1) (layer "F.Cu") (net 1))
 (segment (start 69.03 32.895) (end 70.635 34.5) (width 1) (layer "F.Cu") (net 1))
 (segment (start 33.24 73.38) (end 37.16 77.3) (width 1) (layer "F.Cu") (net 1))
 (segment (start 96.98 31.66) (end 92.83 27.51) (width 1) (layer "F.Cu") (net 1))
 (segment (start 121.655 140) (end 121.955 140.3) (width 1) (layer "F.Cu") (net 1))
 (segment (start 37.16 44) (end 37.16 46.9133) (width 1) (layer "F.Cu") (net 1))
 (segment (start 124.72 70.42) (end 117.84 77.3) (width 1) (layer "F.Cu") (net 1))
 (segment (start 37.16 46.9133) (end 33.24 50.8333) (width 1) (layer "F.Cu") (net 1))
 (segment (start 95.355 147) (end 112.955 147) (width 1) (layer "B.Cu") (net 1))
 (segment (start 112.955 147) (end 116.34 143.615) (width 1) (layer "B.Cu") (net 1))
 (segment (start 38.655 140.3) (end 45.355 147) (width 1) (layer "B.Cu") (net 1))
 (segment (start 45.355 147) (end 65.255 147) (width 1) (layer "B.Cu") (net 1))
 (segment (start 116.34 143.615) (end 116.34 141.34) (width 1) (layer "B.Cu") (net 1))
 (segment (start 115 70.345) (end 115 77.3) (width 1) (layer "B.Cu") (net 1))
 (segment (start 49.5 31.66) (end 37.16 44) (width 1) (layer "B.Cu") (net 1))
 (segment (start 115 77.3) (end 117.84 77.3) (width 1) (layer "B.Cu") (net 1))
 (segment (start 89.7 77.3) (end 115 77.3) (width 1) (layer "B.Cu") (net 1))
 (segment (start 84 83) (end 89.7 77.3) (width 1) (layer "B.Cu") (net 1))
 (segment (start 71.955 140.3) (end 88.655 140.3) (width 1) (layer "B.Cu") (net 1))
 (segment (start 65.255 147) (end 71.955 140.3) (width 1) (layer "B.Cu") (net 1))
 (segment (start 88.655 140.3) (end 95.355 147) (width 1) (layer "B.Cu") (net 1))
 (segment (start 63.68 31.66) (end 49.5 31.66) (width 1) (layer "B.Cu") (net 1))
 (segment (start 116.34 141.34) (end 115 140) (width 1) (layer "B.Cu") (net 1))
 (segment (start 58.075 142.84) (end 58.075 77.34) (width 0.4) (layer "F.Cu") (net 4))
 (segment (start 58.075 77.34) (end 40 59.265) (width 0.4) (layer "F.Cu") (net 4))
 (segment (start 51.15 77.0002) (end 40.3398 66.19) (width 0.4) (layer "F.Cu") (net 14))
 (segment (start 51.15 140) (end 51.15 77.0002) (width 0.4) (layer "F.Cu") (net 14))
 (segment (start 40.3398 66.19) (end 37.16 66.19) (width 0.4) (layer "F.Cu") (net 14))
 (segment (start 52.535 77.34) (end 40 64.805) (width 0.4) (layer "F.Cu") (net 6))
 (segment (start 52.535 142.84) (end 52.535 77.34) (width 0.4) (layer "F.Cu") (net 6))
 (segment (start 114.68 60.65) (end 117.84 60.65) (width 0.4) (layer "F.Cu") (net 25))
 (segment (start 98.38 140) (end 98.38 76.9498) (width 0.4) (layer "F.Cu") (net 25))
 (segment (start 98.38 76.9498) (end 114.68 60.65) (width 0.4) (layer "F.Cu") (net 25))
 (segment (start 96.995 142.84) (end 97.1169 142.718) (width 0.4) (layer "F.Cu") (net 31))
 (segment (start 97.1169 142.718) (end 97.1169 77.1481) (width 0.4) (layer "F.Cu") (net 31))
 (segment (start 97.1169 77.1481) (end 115 59.265) (width 0.4) (layer "F.Cu") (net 31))
 (segment (start 53.92 140) (end 53.92 76.9976) (width 0.4) (layer "F.Cu") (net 13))
 (segment (start 53.92 76.9976) (end 40.3424 63.42) (width 0.4) (layer "F.Cu") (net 13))
 (segment (start 40.3424 63.42) (end 37.16 63.42) (width 0.4) (layer "F.Cu") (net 13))
 (segment (start 40.382767 57.88) (end 59.46 76.957233) (width 0.4) (layer "F.Cu") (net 11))
 (segment (start 37.16 57.88) (end 40.382767 57.88) (width 0.4) (layer "F.Cu") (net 11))
 (segment (start 59.46 76.957233) (end 59.46 140) (width 0.4) (layer "F.Cu") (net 11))
 (segment (start 114.687943 63.42) (end 101.15 76.957943) (width 0.4) (layer "F.Cu") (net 24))
 (segment (start 117.84 63.42) (end 114.687943 63.42) (width 0.4) (layer "F.Cu") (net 24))
 (segment (start 101.15 76.957943) (end 101.15 140) (width 0.4) (layer "F.Cu") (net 24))
 (segment (start 56.69 77.0196) (end 56.69 140) (width 0.4) (layer "F.Cu") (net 12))
 (segment (start 37.16 60.65) (end 40.3204 60.65) (width 0.4) (layer "F.Cu") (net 12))
 (segment (start 40.3204 60.65) (end 56.69 77.0196) (width 0.4) (layer "F.Cu") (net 12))
 (segment (start 117.84 55.11) (end 100.835 55.11) (width 0.4) (layer "B.Cu") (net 19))
 (segment (start 100.835 55.11) (end 63.615 92.33) (width 0.4) (layer "B.Cu") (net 19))
 (segment (start 63.615 92.33) (end 63.615 142.84) (width 0.4) (layer "B.Cu") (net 19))
 (segment (start 99.765 77.27) (end 115 62.035) (width 0.4) (layer "F.Cu") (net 30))
 (segment (start 99.765 142.84) (end 99.765 77.27) (width 0.4) (layer "F.Cu") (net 30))
 (segment (start 65 140) (end 65 92.33) (width 0.4) (layer "B.Cu") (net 16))
 (segment (start 100.835 56.495) (end 115 56.495) (width 0.4) (layer "B.Cu") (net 16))
 (segment (start 65 92.33) (end 100.835 56.495) (width 0.4) (layer "B.Cu") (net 16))
 (segment (start 55.305 142.84) (end 55.305 77.34) (width 0.4) (layer "F.Cu") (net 5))
 (segment (start 55.305 77.34) (end 40 62.035) (width 0.4) (layer "F.Cu") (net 5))
 (segment (start 60.845 142.84) (end 60.845 77.34) (width 0.4) (layer "F.Cu") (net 3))
 (segment (start 60.845 77.34) (end 40 56.495) (width 0.4) (layer "F.Cu") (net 3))
 (segment (start 102.535 142.84) (end 102.535 77.27) (width 0.4) (layer "F.Cu") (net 29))
 (segment (start 102.535 77.27) (end 115 64.805) (width 0.4) (layer "F.Cu") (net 29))
 (segment (start 117.84 57.88) (end 114.664 57.88) (width 0.4) (layer "F.Cu") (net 26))
 (segment (start 96.5152 76.0288) (end 96.5152 139.095) (width 0.4) (layer "F.Cu") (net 26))
 (segment (start 96.5152 139.095) (end 95.61 140) (width 0.4) (layer "F.Cu") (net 26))
 (segment (start 114.664 57.88) (end 96.5152 76.0288) (width 0.4) (layer "F.Cu") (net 26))
 (segment (start 49.6079 103.452) (end 49.6079 140.485) (width 0.4) (layer "B.Cu") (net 20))
 (segment (start 100.72 52.34) (end 49.6079 103.452) (width 0.4) (layer "B.Cu") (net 20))
 (segment (start 47.2525 142.84) (end 46.995 142.84) (width 0.4) (layer "B.Cu") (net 20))
 (segment (start 49.6079 140.485) (end 47.2525 142.84) (width 0.4) (layer "B.Cu") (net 20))
 (segment (start 117.84 52.34) (end 100.72 52.34) (width 0.4) (layer "B.Cu") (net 20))
 (segment (start 100.835 53.725) (end 115 53.725) (width 0.4) (layer "B.Cu") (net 17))
 (segment (start 62.23 140) (end 62.23 92.33) (width 0.4) (layer "B.Cu") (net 17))
 (segment (start 62.23 92.33) (end 100.835 53.725) (width 0.4) (layer "B.Cu") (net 17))
 (segment (start 49.765 77.34) (end 40 67.575) (width 0.4) (layer "F.Cu") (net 7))
 (segment (start 49.765 142.84) (end 49.765 77.34) (width 0.4) (layer "F.Cu") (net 7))
 (segment (start 45.61 140) (end 45.61 81.71) (width 0.4) (layer "F.Cu") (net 15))
 (segment (start 37.16 73.26) (end 37.16 68.96) (width 0.4) (layer "F.Cu") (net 15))
 (segment (start 45.61 81.71) (end 37.16 73.26) (width 0.4) (layer "F.Cu") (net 15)))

